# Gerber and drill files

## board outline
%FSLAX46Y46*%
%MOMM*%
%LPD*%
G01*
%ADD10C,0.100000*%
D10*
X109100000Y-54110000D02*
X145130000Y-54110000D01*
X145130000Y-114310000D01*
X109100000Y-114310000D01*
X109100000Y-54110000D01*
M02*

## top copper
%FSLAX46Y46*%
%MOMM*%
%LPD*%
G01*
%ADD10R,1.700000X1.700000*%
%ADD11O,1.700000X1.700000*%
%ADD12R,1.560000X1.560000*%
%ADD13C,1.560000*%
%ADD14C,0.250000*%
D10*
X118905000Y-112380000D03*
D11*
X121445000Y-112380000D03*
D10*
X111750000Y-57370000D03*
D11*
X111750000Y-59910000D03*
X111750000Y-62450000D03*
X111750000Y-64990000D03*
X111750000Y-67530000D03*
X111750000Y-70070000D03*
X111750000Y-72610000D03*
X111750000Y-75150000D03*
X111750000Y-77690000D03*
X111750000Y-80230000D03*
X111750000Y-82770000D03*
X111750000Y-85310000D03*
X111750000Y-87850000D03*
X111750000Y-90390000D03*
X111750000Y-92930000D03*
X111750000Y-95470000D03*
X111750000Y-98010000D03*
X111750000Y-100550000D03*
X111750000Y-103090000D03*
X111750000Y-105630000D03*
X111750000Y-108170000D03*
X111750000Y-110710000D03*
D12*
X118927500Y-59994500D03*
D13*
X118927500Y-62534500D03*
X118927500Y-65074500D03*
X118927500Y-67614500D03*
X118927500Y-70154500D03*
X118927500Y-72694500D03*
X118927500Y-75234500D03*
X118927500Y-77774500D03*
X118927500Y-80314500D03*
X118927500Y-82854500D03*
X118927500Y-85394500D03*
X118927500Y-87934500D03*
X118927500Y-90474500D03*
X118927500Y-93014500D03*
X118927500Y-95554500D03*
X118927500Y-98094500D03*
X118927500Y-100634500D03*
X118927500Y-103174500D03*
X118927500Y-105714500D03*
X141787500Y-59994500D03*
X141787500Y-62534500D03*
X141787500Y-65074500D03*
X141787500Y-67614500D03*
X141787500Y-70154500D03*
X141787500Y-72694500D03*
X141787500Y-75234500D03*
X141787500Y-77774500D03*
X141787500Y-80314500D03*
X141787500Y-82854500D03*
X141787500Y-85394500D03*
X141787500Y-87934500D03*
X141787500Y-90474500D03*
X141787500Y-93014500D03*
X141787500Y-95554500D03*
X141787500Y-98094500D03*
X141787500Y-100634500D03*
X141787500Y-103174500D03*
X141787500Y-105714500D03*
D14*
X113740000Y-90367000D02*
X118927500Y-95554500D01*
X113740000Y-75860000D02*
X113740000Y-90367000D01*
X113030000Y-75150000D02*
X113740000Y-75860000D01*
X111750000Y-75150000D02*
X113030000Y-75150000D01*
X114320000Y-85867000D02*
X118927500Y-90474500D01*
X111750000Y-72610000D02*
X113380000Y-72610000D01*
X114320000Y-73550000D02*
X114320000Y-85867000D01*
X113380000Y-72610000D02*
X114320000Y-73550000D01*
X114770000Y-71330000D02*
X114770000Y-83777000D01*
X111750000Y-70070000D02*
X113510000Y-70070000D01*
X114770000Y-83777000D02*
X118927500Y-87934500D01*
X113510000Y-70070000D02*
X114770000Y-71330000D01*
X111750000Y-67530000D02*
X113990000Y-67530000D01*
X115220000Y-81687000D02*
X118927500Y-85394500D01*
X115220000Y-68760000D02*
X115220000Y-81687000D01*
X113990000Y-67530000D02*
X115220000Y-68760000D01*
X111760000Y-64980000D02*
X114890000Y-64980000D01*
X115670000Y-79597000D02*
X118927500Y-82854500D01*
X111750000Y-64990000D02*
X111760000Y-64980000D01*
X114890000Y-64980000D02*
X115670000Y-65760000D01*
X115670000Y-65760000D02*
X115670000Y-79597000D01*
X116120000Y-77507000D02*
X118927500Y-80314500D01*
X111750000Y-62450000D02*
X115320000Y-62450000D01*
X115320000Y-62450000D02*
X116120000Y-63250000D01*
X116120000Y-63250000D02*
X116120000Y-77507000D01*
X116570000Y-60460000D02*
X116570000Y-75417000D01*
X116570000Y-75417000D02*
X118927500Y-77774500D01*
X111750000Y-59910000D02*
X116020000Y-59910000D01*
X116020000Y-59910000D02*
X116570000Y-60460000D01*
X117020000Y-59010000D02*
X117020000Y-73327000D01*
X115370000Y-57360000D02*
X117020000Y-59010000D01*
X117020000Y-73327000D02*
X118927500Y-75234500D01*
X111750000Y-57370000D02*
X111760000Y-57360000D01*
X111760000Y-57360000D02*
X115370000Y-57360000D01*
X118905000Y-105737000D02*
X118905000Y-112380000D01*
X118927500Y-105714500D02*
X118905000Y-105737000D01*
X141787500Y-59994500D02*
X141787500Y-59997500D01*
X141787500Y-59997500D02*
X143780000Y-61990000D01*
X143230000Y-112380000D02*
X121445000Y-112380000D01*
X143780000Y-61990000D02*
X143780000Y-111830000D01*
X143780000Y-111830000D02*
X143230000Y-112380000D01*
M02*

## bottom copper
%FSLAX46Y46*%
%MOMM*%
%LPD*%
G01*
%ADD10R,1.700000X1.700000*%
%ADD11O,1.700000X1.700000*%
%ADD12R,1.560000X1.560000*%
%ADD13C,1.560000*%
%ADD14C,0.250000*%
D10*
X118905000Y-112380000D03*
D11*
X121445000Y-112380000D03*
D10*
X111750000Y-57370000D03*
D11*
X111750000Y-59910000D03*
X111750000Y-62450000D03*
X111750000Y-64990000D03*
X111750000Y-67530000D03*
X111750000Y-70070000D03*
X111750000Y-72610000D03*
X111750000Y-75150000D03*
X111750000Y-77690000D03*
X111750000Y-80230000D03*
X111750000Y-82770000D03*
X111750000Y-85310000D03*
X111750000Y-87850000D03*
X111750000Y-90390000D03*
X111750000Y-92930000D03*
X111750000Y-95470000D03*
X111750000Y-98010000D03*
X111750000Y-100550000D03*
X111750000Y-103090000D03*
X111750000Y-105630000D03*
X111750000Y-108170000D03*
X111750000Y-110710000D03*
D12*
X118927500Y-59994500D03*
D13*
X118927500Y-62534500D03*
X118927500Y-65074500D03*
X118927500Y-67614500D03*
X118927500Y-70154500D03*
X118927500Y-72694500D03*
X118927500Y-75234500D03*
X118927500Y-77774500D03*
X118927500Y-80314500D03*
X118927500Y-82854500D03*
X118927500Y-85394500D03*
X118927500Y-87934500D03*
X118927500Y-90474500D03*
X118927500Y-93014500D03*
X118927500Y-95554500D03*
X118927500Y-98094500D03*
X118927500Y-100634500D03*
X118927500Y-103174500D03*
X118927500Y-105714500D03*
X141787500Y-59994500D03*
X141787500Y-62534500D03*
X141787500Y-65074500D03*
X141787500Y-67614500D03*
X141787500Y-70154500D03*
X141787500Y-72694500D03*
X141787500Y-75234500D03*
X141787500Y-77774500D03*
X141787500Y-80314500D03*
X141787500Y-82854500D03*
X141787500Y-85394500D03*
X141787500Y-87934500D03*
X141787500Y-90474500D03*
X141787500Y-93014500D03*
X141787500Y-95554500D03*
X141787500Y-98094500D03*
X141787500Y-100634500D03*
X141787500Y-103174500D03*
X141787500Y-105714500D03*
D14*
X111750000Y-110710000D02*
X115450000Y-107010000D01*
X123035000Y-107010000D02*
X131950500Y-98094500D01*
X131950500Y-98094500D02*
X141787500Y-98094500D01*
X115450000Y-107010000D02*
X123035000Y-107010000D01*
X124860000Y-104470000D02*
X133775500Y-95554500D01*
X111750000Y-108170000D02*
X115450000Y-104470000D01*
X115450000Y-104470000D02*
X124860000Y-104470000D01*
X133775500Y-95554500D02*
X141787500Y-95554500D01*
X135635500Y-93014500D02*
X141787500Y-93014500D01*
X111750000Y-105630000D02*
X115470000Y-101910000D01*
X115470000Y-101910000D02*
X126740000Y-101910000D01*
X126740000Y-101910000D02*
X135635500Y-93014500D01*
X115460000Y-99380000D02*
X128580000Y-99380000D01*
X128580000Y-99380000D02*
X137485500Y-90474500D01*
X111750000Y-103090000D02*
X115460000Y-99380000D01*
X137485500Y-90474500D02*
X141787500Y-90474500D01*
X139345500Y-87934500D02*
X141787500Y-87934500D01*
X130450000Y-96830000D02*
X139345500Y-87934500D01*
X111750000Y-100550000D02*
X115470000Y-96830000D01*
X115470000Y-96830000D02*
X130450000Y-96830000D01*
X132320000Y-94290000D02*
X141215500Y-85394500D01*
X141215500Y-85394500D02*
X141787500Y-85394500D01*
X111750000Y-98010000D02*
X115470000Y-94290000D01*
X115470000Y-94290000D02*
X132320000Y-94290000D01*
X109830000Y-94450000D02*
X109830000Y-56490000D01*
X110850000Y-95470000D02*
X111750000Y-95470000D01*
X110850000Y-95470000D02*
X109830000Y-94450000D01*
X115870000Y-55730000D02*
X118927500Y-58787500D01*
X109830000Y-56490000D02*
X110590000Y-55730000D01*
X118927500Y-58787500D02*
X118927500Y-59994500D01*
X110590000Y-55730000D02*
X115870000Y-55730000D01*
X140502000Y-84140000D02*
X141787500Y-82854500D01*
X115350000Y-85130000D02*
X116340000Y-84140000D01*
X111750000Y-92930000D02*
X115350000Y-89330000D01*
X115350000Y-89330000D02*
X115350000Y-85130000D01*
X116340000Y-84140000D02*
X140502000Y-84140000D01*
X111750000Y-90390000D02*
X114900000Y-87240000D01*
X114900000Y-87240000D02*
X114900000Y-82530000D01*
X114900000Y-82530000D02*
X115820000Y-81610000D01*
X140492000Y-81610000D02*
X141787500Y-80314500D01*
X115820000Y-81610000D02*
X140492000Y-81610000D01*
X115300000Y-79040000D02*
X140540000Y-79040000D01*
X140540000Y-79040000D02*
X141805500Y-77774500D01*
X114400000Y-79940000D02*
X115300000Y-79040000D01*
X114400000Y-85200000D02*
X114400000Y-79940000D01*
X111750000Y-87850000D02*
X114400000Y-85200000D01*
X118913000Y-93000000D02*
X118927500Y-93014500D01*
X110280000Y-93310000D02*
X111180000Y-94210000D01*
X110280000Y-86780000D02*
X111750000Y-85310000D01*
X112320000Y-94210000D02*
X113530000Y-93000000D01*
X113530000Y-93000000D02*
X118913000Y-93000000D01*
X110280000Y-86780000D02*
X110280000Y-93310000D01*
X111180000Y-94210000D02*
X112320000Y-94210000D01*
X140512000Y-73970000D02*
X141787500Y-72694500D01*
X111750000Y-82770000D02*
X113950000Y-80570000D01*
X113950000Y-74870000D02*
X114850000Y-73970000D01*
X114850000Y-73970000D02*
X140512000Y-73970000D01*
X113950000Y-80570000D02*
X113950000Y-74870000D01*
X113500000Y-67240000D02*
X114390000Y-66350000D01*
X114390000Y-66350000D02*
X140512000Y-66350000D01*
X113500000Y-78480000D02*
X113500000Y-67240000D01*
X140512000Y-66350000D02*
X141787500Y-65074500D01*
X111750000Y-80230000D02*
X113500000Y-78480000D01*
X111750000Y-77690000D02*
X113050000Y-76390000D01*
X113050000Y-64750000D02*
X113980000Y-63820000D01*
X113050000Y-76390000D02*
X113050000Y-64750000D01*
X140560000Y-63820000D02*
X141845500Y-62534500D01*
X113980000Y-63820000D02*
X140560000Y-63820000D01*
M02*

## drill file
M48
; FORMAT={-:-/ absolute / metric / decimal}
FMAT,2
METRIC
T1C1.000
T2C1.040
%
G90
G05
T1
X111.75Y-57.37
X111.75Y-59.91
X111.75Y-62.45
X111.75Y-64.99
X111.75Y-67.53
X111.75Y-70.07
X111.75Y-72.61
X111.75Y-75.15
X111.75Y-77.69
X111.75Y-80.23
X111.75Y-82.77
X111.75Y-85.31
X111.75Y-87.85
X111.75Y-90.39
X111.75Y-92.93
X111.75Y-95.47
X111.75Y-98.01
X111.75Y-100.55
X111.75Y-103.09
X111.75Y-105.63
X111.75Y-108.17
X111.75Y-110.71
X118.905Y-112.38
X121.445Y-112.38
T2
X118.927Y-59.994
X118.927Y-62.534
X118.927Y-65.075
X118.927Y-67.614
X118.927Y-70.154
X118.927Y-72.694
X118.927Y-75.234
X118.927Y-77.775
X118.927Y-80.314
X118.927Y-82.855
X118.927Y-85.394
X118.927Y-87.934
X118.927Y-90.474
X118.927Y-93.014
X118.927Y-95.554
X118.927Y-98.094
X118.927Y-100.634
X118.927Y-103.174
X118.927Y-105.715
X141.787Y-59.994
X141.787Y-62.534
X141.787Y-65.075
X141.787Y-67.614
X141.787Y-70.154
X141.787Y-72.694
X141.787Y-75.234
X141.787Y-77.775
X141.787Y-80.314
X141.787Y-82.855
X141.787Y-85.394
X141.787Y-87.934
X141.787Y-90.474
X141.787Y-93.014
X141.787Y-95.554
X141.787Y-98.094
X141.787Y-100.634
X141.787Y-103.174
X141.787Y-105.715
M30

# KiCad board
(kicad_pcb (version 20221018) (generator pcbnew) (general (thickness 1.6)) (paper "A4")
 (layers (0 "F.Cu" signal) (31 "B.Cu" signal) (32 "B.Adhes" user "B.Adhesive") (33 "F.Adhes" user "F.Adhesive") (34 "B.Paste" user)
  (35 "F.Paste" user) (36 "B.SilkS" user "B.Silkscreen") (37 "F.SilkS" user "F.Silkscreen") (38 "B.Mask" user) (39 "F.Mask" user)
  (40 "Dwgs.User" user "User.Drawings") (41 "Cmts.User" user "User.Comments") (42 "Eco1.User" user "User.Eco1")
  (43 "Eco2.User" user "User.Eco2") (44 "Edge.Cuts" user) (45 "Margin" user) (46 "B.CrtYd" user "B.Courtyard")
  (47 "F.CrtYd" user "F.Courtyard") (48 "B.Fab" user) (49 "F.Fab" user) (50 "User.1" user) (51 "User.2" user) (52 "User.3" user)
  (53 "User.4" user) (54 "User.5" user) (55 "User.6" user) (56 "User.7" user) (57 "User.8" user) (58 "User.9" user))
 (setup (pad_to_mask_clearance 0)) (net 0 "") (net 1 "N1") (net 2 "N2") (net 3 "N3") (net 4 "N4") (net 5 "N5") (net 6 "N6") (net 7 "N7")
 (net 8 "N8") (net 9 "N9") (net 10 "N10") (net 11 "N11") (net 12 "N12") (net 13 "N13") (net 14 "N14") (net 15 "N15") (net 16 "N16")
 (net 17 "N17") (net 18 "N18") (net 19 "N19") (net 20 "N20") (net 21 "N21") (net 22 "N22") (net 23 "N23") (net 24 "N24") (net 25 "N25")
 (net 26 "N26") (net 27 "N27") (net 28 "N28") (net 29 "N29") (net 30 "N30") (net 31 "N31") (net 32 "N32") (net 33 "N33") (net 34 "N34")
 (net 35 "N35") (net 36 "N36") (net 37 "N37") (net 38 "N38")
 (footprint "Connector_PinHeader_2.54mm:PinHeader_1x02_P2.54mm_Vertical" (layer "F.Cu") (at 118.905 112.38 90)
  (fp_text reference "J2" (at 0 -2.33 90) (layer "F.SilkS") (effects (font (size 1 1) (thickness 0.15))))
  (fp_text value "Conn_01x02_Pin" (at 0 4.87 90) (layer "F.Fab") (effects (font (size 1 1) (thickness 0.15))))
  (pad "1" thru_hole rect (at 0 0 90) (size 1.7 1.7) (drill 1) (layers "*.Cu" "*.Mask") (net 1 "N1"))
  (pad "2" thru_hole oval (at 0 2.54 90) (size 1.7 1.7) (drill 1) (layers "*.Cu" "*.Mask") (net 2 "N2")))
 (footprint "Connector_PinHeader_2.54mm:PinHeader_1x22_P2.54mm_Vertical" (layer "F.Cu") (at 111.75 57.37)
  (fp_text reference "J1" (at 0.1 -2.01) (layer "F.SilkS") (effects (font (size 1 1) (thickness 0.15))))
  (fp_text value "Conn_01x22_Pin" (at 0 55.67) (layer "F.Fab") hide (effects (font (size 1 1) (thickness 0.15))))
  (pad "1" thru_hole rect (at 0 0) (size 1.7 1.7) (drill 1) (layers "*.Cu" "*.Mask") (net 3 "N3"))
  (pad "2" thru_hole oval (at 0 2.54) (size 1.7 1.7) (drill 1) (layers "*.Cu" "*.Mask") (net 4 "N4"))
  (pad "3" thru_hole oval (at 0 5.08) (size 1.7 1.7) (drill 1) (layers "*.Cu" "*.Mask") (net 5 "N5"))
  (pad "4" thru_hole oval (at 0 7.62) (size 1.7 1.7) (drill 1) (layers "*.Cu" "*.Mask") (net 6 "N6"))
  (pad "5" thru_hole oval (at 0 10.16) (size 1.7 1.7) (drill 1) (layers "*.Cu" "*.Mask") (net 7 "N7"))
  (pad "6" thru_hole oval (at 0 12.7) (size 1.7 1.7) (drill 1) (layers "*.Cu" "*.Mask") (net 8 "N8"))
  (pad "7" thru_hole oval (at 0 15.24) (size 1.7 1.7) (drill 1) (layers "*.Cu" "*.Mask") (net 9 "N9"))
  (pad "8" thru_hole oval (at 0 17.78) (size 1.7 1.7) (drill 1) (layers "*.Cu" "*.Mask") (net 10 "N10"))
  (pad "9" thru_hole oval (at 0 20.32) (size 1.7 1.7) (drill 1) (layers "*.Cu" "*.Mask") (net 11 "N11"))
  (pad "10" thru_hole oval (at 0 22.86) (size 1.7 1.7) (drill 1) (layers "*.Cu" "*.Mask") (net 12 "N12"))
  (pad "11" thru_hole oval (at 0 25.4) (size 1.7 1.7) (drill 1) (layers "*.Cu" "*.Mask") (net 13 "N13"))
  (pad "12" thru_hole oval (at 0 27.94) (size 1.7 1.7) (drill 1) (layers "*.Cu" "*.Mask") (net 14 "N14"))
  (pad "13" thru_hole oval (at 0 30.48) (size 1.7 1.7) (drill 1) (layers "*.Cu" "*.Mask") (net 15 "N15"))
  (pad "14" thru_hole oval (at 0 33.02) (size 1.7 1.7) (drill 1) (layers "*.Cu" "*.Mask") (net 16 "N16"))
  (pad "15" thru_hole oval (at 0 35.56) (size 1.7 1.7) (drill 1) (layers "*.Cu" "*.Mask") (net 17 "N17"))
  (pad "16" thru_hole oval (at 0 38.1) (size 1.7 1.7) (drill 1) (layers "*.Cu" "*.Mask") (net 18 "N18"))
  (pad "17" thru_hole oval (at 0 40.64) (size 1.7 1.7) (drill 1) (layers "*.Cu" "*.Mask") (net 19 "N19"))
  (pad "18" thru_hole oval (at 0 43.18) (size 1.7 1.7) (drill 1) (layers "*.Cu" "*.Mask") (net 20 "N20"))
  (pad "19" thru_hole oval (at 0 45.72) (size 1.7 1.7) (drill 1) (layers "*.Cu" "*.Mask") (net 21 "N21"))
  (pad "20" thru_hole oval (at 0 48.26) (size 1.7 1.7) (drill 1) (layers "*.Cu" "*.Mask") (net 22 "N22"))
  (pad "21" thru_hole oval (at 0 50.8) (size 1.7 1.7) (drill 1) (layers "*.Cu" "*.Mask") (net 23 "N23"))
  (pad "22" thru_hole oval (at 0 53.34) (size 1.7 1.7) (drill 1) (layers "*.Cu" "*.Mask") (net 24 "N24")))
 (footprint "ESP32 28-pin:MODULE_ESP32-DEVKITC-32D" (layer "F.Cu") (at 131.6275 79.7545)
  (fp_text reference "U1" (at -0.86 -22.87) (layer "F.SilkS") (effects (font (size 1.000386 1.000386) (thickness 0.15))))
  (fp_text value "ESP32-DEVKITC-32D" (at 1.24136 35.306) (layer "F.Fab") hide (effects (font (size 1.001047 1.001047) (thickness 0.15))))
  (pad "J2-1" thru_hole rect (at -12.7 -19.76) (size 1.56 1.56) (drill 1.04) (layers "*.Cu" "*.Mask") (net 18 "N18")
   (solder_mask_margin 0.102))
  (pad "J2-2" thru_hole circle (at -12.7 -17.22) (size 1.56 1.56) (drill 1.04) (layers "*.Cu" "*.Mask") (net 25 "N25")
   (solder_mask_margin 0.102))
  (pad "J2-3" thru_hole circle (at -12.7 -14.68) (size 1.56 1.56) (drill 1.04) (layers "*.Cu" "*.Mask") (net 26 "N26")
   (solder_mask_margin 0.102))
  (pad "J2-4" thru_hole circle (at -12.7 -12.14) (size 1.56 1.56) (drill 1.04) (layers "*.Cu" "*.Mask") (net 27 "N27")
   (solder_mask_margin 0.102))
  (pad "J2-5" thru_hole circle (at -12.7 -9.6) (size 1.56 1.56) (drill 1.04) (layers "*.Cu" "*.Mask") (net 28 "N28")
   (solder_mask_margin 0.102))
  (pad "J2-6" thru_hole circle (at -12.7 -7.06) (size 1.56 1.56) (drill 1.04) (layers "*.Cu" "*.Mask") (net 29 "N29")
   (solder_mask_margin 0.102))
  (pad "J2-7" thru_hole circle (at -12.7 -4.52) (size 1.56 1.56) (drill 1.04) (layers "*.Cu" "*.Mask") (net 3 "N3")
   (solder_mask_margin 0.102))
  (pad "J2-8" thru_hole circle (at -12.7 -1.98) (size 1.56 1.56) (drill 1.04) (layers "*.Cu" "*.Mask") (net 4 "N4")
   (solder_mask_margin 0.102))
  (pad "J2-9" thru_hole circle (at -12.7 0.56) (size 1.56 1.56) (drill 1.04) (layers "*.Cu" "*.Mask") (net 5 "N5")
   (solder_mask_margin 0.102))
  (pad "J2-10" thru_hole circle (at -12.7 3.1) (size 1.56 1.56) (drill 1.04) (layers "*.Cu" "*.Mask") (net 6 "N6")
   (solder_mask_margin 0.102))
  (pad "J2-11" thru_hole circle (at -12.7 5.64) (size 1.56 1.56) (drill 1.04) (layers "*.Cu" "*.Mask") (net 7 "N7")
   (solder_mask_margin 0.102))
  (pad "J2-12" thru_hole circle (at -12.7 8.18) (size 1.56 1.56) (drill 1.04) (layers "*.Cu" "*.Mask") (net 8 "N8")
   (solder_mask_margin 0.102))
  (pad "J2-13" thru_hole circle (at -12.7 10.72) (size 1.56 1.56) (drill 1.04) (layers "*.Cu" "*.Mask") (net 9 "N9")
   (solder_mask_margin 0.102))
  (pad "J2-14" thru_hole circle (at -12.7 13.26) (size 1.56 1.56) (drill 1.04) (layers "*.Cu" "*.Mask") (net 14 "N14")
   (solder_mask_margin 0.102))
  (pad "J2-15" thru_hole circle (at -12.7 15.8) (size 1.56 1.56) (drill 1.04) (layers "*.Cu" "*.Mask") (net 10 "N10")
   (solder_mask_margin 0.102))
  (pad "J2-16" thru_hole circle (at -12.7 18.34) (size 1.56 1.56) (drill 1.04) (layers "*.Cu" "*.Mask") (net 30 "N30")
   (solder_mask_margin 0.102))
  (pad "J2-17" thru_hole circle (at -12.7 20.88) (size 1.56 1.56) (drill 1.04) (layers "*.Cu" "*.Mask") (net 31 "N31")
   (solder_mask_margin 0.102))
  (pad "J2-18" thru_hole circle (at -12.7 23.42) (size 1.56 1.56) (drill 1.04) (layers "*.Cu" "*.Mask") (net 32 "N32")
   (solder_mask_margin 0.102))
  (pad "J2-19" thru_hole circle (at -12.7 25.96) (size 1.56 1.56) (drill 1.04) (layers "*.Cu" "*.Mask") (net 1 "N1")
   (solder_mask_margin 0.102))
  (pad "J3-1" thru_hole circle (at 10.16 -19.76) (size 1.56 1.56) (drill 1.04) (layers "*.Cu" "*.Mask") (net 2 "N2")
   (solder_mask_margin 0.102))
  (pad "J3-2" thru_hole circle (at 10.16 -17.22) (size 1.56 1.56) (drill 1.04) (layers "*.Cu" "*.Mask") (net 11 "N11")
   (solder_mask_margin 0.102))
  (pad "J3-3" thru_hole circle (at 10.16 -14.68) (size 1.56 1.56) (drill 1.04) (layers "*.Cu" "*.Mask") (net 12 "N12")
   (solder_mask_margin 0.102))
  (pad "J3-4" thru_hole circle (at 10.16 -12.14) (size 1.56 1.56) (drill 1.04) (layers "*.Cu" "*.Mask") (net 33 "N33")
   (solder_mask_margin 0.102))
  (pad "J3-5" thru_hole circle (at 10.16 -9.6) (size 1.56 1.56) (drill 1.04) (layers "*.Cu" "*.Mask") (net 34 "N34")
   (solder_mask_margin 0.102))
  (pad "J3-6" thru_hole circle (at 10.16 -7.06) (size 1.56 1.56) (drill 1.04) (layers "*.Cu" "*.Mask") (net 13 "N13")
   (solder_mask_margin 0.102))
  (pad "J3-7" thru_hole circle (at 10.16 -4.52) (size 1.56 1.56) (drill 1.04) (layers "*.Cu" "*.Mask") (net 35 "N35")
   (solder_mask_margin 0.102))
  (pad "J3-8" thru_hole circle (at 10.16 -1.98) (size 1.56 1.56) (drill 1.04) (layers "*.Cu" "*.Mask") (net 15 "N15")
   (solder_mask_margin 0.102))
  (pad "J3-9" thru_hole circle (at 10.16 0.56) (size 1.56 1.56) (drill 1.04) (layers "*.Cu" "*.Mask") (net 16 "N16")
   (solder_mask_margin 0.102))
  (pad "J3-10" thru_hole circle (at 10.16 3.1) (size 1.56 1.56) (drill 1.04) (layers "*.Cu" "*.Mask") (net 17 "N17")
   (solder_mask_margin 0.102))
  (pad "J3-11" thru_hole circle (at 10.16 5.64) (size 1.56 1.56) (drill 1.04) (layers "*.Cu" "*.Mask") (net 19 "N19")
   (solder_mask_margin 0.102))
  (pad "J3-12" thru_hole circle (at 10.16 8.18) (size 1.56 1.56) (drill 1.04) (layers "*.Cu" "*.Mask") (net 20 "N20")
   (solder_mask_margin 0.102))
  (pad "J3-13" thru_hole circle (at 10.16 10.72) (size 1.56 1.56) (drill 1.04) (layers "*.Cu" "*.Mask") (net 21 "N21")
   (solder_mask_margin 0.102))
  (pad "J3-14" thru_hole circle (at 10.16 13.26) (size 1.56 1.56) (drill 1.04) (layers "*.Cu" "*.Mask") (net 22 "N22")
   (solder_mask_margin 0.102))
  (pad "J3-15" thru_hole circle (at 10.16 15.8) (size 1.56 1.56) (drill 1.04) (layers "*.Cu" "*.Mask") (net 23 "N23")
   (solder_mask_margin 0.102))
  (pad "J3-16" thru_hole circle (at 10.16 18.34) (size 1.56 1.56) (drill 1.04) (layers "*.Cu" "*.Mask") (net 24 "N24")
   (solder_mask_margin 0.102))
  (pad "J3-17" thru_hole circle (at 10.16 20.88) (size 1.56 1.56) (drill 1.04) (layers "*.Cu" "*.Mask") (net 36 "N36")
   (solder_mask_margin 0.102))
  (pad "J3-18" thru_hole circle (at 10.16 23.42) (size 1.56 1.56) (drill 1.04) (layers "*.Cu" "*.Mask") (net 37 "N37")
   (solder_mask_margin 0.102))
  (pad "J3-19" thru_hole circle (at 10.16 25.96) (size 1.56 1.56) (drill 1.04) (layers "*.Cu" "*.Mask") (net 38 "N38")
   (solder_mask_margin 0.102)))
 (gr_rect (start 109.1 54.11) (end 145.13 114.31) (stroke (width 0.1) (type default)) (fill none) (layer "Edge.Cuts"))
 (segment (start 111.75 110.71) (end 115.45 107.01) (width 0.25) (layer "B.Cu") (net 24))
 (segment (start 123.035 107.01) (end 131.9505 98.0945) (width 0.25) (layer "B.Cu") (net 24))
 (segment (start 131.9505 98.0945) (end 141.7875 98.0945) (width 0.25) (layer "B.Cu") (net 24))
 (segment (start 115.45 107.01) (end 123.035 107.01) (width 0.25) (layer "B.Cu") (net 24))
 (segment (start 124.86 104.47) (end 133.7755 95.5545) (width 0.25) (layer "B.Cu") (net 23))
 (segment (start 111.75 108.17) (end 115.45 104.47) (width 0.25) (layer "B.Cu") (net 23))
 (segment (start 115.45 104.47) (end 124.86 104.47) (width 0.25) (layer "B.Cu") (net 23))
 (segment (start 133.7755 95.5545) (end 141.7875 95.5545) (width 0.25) (layer "B.Cu") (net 23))
 (segment (start 135.6355 93.0145) (end 141.7875 93.0145) (width 0.25) (layer "B.Cu") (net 22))
 (segment (start 111.75 105.63) (end 115.47 101.91) (width 0.25) (layer "B.Cu") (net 22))
 (segment (start 115.47 101.91) (end 126.74 101.91) (width 0.25) (layer "B.Cu") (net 22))
 (segment (start 126.74 101.91) (end 135.6355 93.0145) (width 0.25) (layer "B.Cu") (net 22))
 (segment (start 115.46 99.38) (end 128.58 99.38) (width 0.25) (layer "B.Cu") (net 21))
 (segment (start 128.58 99.38) (end 137.4855 90.4745) (width 0.25) (layer "B.Cu") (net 21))
 (segment (start 111.75 103.09) (end 115.46 99.38) (width 0.25) (layer "B.Cu") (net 21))
 (segment (start 137.4855 90.4745) (end 141.7875 90.4745) (width 0.25) (layer "B.Cu") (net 21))
 (segment (start 139.3455 87.9345) (end 141.7875 87.9345) (width 0.25) (layer "B.Cu") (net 20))
 (segment (start 130.45 96.83) (end 139.3455 87.9345) (width 0.25) (layer "B.Cu") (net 20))
 (segment (start 111.75 100.55) (end 115.47 96.83) (width 0.25) (layer "B.Cu") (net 20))
 (segment (start 115.47 96.83) (end 130.45 96.83) (width 0.25) (layer "B.Cu") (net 20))
 (segment (start 132.32 94.29) (end 141.2155 85.3945) (width 0.25) (layer "B.Cu") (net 19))
 (segment (start 141.2155 85.3945) (end 141.7875 85.3945) (width 0.25) (layer "B.Cu") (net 19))
 (segment (start 111.75 98.01) (end 115.47 94.29) (width 0.25) (layer "B.Cu") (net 19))
 (segment (start 115.47 94.29) (end 132.32 94.29) (width 0.25) (layer "B.Cu") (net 19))
 (segment (start 109.83 94.45) (end 109.83 56.49) (width 0.25) (layer "B.Cu") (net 18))
 (segment (start 110.85 95.47) (end 111.75 95.47) (width 0.25) (layer "B.Cu") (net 18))
 (segment (start 110.85 95.47) (end 109.83 94.45) (width 0.25) (layer "B.Cu") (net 18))
 (segment (start 115.87 55.73) (end 118.9275 58.7875) (width 0.25) (layer "B.Cu") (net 18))
 (segment (start 109.83 56.49) (end 110.59 55.73) (width 0.25) (layer "B.Cu") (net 18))
 (segment (start 118.9275 58.7875) (end 118.9275 59.9945) (width 0.25) (layer "B.Cu") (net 18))
 (segment (start 110.59 55.73) (end 115.87 55.73) (width 0.25) (layer "B.Cu") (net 18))
 (segment (start 140.502 84.14) (end 141.7875 82.8545) (width 0.25) (layer "B.Cu") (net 17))
 (segment (start 115.35 85.13) (end 116.34 84.14) (width 0.25) (layer "B.Cu") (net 17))
 (segment (start 111.75 92.93) (end 115.35 89.33) (width 0.25) (layer "B.Cu") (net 17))
 (segment (start 115.35 89.33) (end 115.35 85.13) (width 0.25) (layer "B.Cu") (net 17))
 (segment (start 116.34 84.14) (end 140.502 84.14) (width 0.25) (layer "B.Cu") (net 17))
 (segment (start 111.75 90.39) (end 114.9 87.24) (width 0.25) (layer "B.Cu") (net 16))
 (segment (start 114.9 87.24) (end 114.9 82.53) (width 0.25) (layer "B.Cu") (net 16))
 (segment (start 114.9 82.53) (end 115.82 81.61) (width 0.25) (layer "B.Cu") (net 16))
 (segment (start 140.492 81.61) (end 141.7875 80.3145) (width 0.25) (layer "B.Cu") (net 16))
 (segment (start 115.82 81.61) (end 140.492 81.61) (width 0.25) (layer "B.Cu") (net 16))
 (segment (start 115.3 79.04) (end 140.54 79.04) (width 0.25) (layer "B.Cu") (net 15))
 (segment (start 140.54 79.04) (end 141.8055 77.7745) (width 0.25) (layer "B.Cu") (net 15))
 (segment (start 114.4 79.94) (end 115.3 79.04) (width 0.25) (layer "B.Cu") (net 15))
 (segment (start 114.4 85.2) (end 114.4 79.94) (width 0.25) (layer "B.Cu") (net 15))
 (segment (start 111.75 87.85) (end 114.4 85.2) (width 0.25) (layer "B.Cu") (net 15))
 (segment (start 118.913 93) (end 118.9275 93.0145) (width 0.25) (layer "B.Cu") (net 14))
 (segment (start 110.28 93.31) (end 111.18 94.21) (width 0.25) (layer "B.Cu") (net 14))
 (segment (start 110.28 86.78) (end 111.75 85.31) (width 0.25) (layer "B.Cu") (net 14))
 (segment (start 112.32 94.21) (end 113.53 93) (width 0.25) (layer "B.Cu") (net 14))
 (segment (start 113.53 93) (end 118.913 93) (width 0.25) (layer "B.Cu") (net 14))
 (segment (start 110.28 86.78) (end 110.28 93.31) (width 0.25) (layer "B.Cu") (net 14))
 (segment (start 111.18 94.21) (end 112.32 94.21) (width 0.25) (layer "B.Cu") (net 14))
 (segment (start 140.512 73.97) (end 141.7875 72.6945) (width 0.25) (layer "B.Cu") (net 13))
 (segment (start 111.75 82.77) (end 113.95 80.57) (width 0.25) (layer "B.Cu") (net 13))
 (segment (start 113.95 74.87) (end 114.85 73.97) (width 0.25) (layer "B.Cu") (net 13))
 (segment (start 114.85 73.97) (end 140.512 73.97) (width 0.25) (layer "B.Cu") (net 13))
 (segment (start 113.95 80.57) (end 113.95 74.87) (width 0.25) (layer "B.Cu") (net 13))
 (segment (start 113.5 67.24) (end 114.39 66.35) (width 0.25) (layer "B.Cu") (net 12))
 (segment (start 114.39 66.35) (end 140.512 66.35) (width 0.25) (layer "B.Cu") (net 12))
 (segment (start 113.5 78.48) (end 113.5 67.24) (width 0.25) (layer "B.Cu") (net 12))
 (segment (start 140.512 66.35) (end 141.7875 65.0745) (width 0.25) (layer "B.Cu") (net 12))
 (segment (start 111.75 80.23) (end 113.5 78.48) (width 0.25) (layer "B.Cu") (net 12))
 (segment (start 111.75 77.69) (end 113.05 76.39) (width 0.25) (layer "B.Cu") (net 11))
 (segment (start 113.05 64.75) (end 113.98 63.82) (width 0.25) (layer "B.Cu") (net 11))
 (segment (start 113.05 76.39) (end 113.05 64.75) (width 0.25) (layer "B.Cu") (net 11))
 (segment (start 140.56 63.82) (end 141.8455 62.5345) (width 0.25) (layer "B.Cu") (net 11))
 (segment (start 113.98 63.82) (end 140.56 63.82) (width 0.25) (layer "B.Cu") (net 11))
 (segment (start 113.74 90.367) (end 118.9275 95.5545) (width 0.25) (layer "F.Cu") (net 10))
 (segment (start 113.74 75.86) (end 113.74 90.367) (width 0.25) (layer "F.Cu") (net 10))
 (segment (start 113.03 75.15) (end 113.74 75.86) (width 0.25) (layer "F.Cu") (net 10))
 (segment (start 111.75 75.15) (end 113.03 75.15) (width 0.25) (layer "F.Cu") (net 10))
 (segment (start 114.32 85.867) (end 118.9275 90.4745) (width 0.25) (layer "F.Cu") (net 9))
 (segment (start 111.75 72.61) (end 113.38 72.61) (width 0.25) (layer "F.Cu") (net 9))
 (segment (start 114.32 73.55) (end 114.32 85.867) (width 0.25) (layer "F.Cu") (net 9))
 (segment (start 113.38 72.61) (end 114.32 73.55) (width 0.25) (layer "F.Cu") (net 9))
 (segment (start 114.77 71.33) (end 114.77 83.777) (width 0.25) (layer "F.Cu") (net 8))
 (segment (start 111.75 70.07) (end 113.51 70.07) (width 0.25) (layer "F.Cu") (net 8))
 (segment (start 114.77 83.777) (end 118.9275 87.9345) (width 0.25) (layer "F.Cu") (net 8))
 (segment (start 113.51 70.07) (end 114.77 71.33) (width 0.25) (layer "F.Cu") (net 8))
 (segment (start 111.75 67.53) (end 113.99 67.53) (width 0.25) (layer "F.Cu") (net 7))
 (segment (start 115.22 81.687) (end 118.9275 85.3945) (width 0.25) (layer "F.Cu") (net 7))
 (segment (start 115.22 68.76) (end 115.22 81.687) (width 0.25) (layer "F.Cu") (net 7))
 (segment (start 113.99 67.53) (end 115.22 68.76) (width 0.25) (layer "F.Cu") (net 7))
 (segment (start 111.76 64.98) (end 114.89 64.98) (width 0.25) (layer "F.Cu") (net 6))
 (segment (start 115.67 79.597) (end 118.9275 82.8545) (width 0.25) (layer "F.Cu") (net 6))
 (segment (start 111.75 64.99) (end 111.76 64.98) (width 0.25) (layer "F.Cu") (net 6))
 (segment (start 114.89 64.98) (end 115.67 65.76) (width 0.25) (layer "F.Cu") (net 6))
 (segment (start 115.67 65.76) (end 115.67 79.597) (width 0.25) (layer "F.Cu") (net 6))
 (segment (start 116.12 77.507) (end 118.9275 80.3145) (width 0.25) (layer "F.Cu") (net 5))
 (segment (start 111.75 62.45) (end 115.32 62.45) (width 0.25) (layer "F.Cu") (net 5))
 (segment (start 115.32 62.45) (end 116.12 63.25) (width 0.25) (layer "F.Cu") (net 5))
 (segment (start 116.12 63.25) (end 116.12 77.507) (width 0.25) (layer "F.Cu") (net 5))
 (segment (start 116.57 60.46) (end 116.57 75.417) (width 0.25) (layer "F.Cu") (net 4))
 (segment (start 116.57 75.417) (end 118.9275 77.7745) (width 0.25) (layer "F.Cu") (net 4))
 (segment (start 111.75 59.91) (end 116.02 59.91) (width 0.25) (layer "F.Cu") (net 4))
 (segment (start 116.02 59.91) (end 116.57 60.46) (width 0.25) (layer "F.Cu") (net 4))
 (segment (start 117.02 59.01) (end 117.02 73.327) (width 0.25) (layer "F.Cu") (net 3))
 (segment (start 115.37 57.36) (end 117.02 59.01) (width 0.25) (layer "F.Cu") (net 3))
 (segment (start 117.02 73.327) (end 118.9275 75.2345) (width 0.25) (layer "F.Cu") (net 3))
 (segment (start 111.75 57.37) (end 111.76 57.36) (width 0.25) (layer "F.Cu") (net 3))
 (segment (start 111.76 57.36) (end 115.37 57.36) (width 0.25) (layer "F.Cu") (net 3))
 (segment (start 118.905 105.737) (end 118.905 112.38) (width 0.25) (layer "F.Cu") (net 1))
 (segment (start 118.9275 105.7145) (end 118.905 105.737) (width 0.25) (layer "F.Cu") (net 1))
 (segment (start 141.7875 59.9945) (end 141.7875 59.9975) (width 0.25) (layer "F.Cu") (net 2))
 (segment (start 141.7875 59.9975) (end 143.78 61.99) (width 0.25) (layer "F.Cu") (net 2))
 (segment (start 143.23 112.38) (end 121.445 112.38) (width 0.25) (layer "F.Cu") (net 2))
 (segment (start 143.78 61.99) (end 143.78 111.83) (width 0.25) (layer "F.Cu") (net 2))
 (segment (start 143.78 111.83) (end 143.23 112.38) (width 0.25) (layer "F.Cu") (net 2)))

